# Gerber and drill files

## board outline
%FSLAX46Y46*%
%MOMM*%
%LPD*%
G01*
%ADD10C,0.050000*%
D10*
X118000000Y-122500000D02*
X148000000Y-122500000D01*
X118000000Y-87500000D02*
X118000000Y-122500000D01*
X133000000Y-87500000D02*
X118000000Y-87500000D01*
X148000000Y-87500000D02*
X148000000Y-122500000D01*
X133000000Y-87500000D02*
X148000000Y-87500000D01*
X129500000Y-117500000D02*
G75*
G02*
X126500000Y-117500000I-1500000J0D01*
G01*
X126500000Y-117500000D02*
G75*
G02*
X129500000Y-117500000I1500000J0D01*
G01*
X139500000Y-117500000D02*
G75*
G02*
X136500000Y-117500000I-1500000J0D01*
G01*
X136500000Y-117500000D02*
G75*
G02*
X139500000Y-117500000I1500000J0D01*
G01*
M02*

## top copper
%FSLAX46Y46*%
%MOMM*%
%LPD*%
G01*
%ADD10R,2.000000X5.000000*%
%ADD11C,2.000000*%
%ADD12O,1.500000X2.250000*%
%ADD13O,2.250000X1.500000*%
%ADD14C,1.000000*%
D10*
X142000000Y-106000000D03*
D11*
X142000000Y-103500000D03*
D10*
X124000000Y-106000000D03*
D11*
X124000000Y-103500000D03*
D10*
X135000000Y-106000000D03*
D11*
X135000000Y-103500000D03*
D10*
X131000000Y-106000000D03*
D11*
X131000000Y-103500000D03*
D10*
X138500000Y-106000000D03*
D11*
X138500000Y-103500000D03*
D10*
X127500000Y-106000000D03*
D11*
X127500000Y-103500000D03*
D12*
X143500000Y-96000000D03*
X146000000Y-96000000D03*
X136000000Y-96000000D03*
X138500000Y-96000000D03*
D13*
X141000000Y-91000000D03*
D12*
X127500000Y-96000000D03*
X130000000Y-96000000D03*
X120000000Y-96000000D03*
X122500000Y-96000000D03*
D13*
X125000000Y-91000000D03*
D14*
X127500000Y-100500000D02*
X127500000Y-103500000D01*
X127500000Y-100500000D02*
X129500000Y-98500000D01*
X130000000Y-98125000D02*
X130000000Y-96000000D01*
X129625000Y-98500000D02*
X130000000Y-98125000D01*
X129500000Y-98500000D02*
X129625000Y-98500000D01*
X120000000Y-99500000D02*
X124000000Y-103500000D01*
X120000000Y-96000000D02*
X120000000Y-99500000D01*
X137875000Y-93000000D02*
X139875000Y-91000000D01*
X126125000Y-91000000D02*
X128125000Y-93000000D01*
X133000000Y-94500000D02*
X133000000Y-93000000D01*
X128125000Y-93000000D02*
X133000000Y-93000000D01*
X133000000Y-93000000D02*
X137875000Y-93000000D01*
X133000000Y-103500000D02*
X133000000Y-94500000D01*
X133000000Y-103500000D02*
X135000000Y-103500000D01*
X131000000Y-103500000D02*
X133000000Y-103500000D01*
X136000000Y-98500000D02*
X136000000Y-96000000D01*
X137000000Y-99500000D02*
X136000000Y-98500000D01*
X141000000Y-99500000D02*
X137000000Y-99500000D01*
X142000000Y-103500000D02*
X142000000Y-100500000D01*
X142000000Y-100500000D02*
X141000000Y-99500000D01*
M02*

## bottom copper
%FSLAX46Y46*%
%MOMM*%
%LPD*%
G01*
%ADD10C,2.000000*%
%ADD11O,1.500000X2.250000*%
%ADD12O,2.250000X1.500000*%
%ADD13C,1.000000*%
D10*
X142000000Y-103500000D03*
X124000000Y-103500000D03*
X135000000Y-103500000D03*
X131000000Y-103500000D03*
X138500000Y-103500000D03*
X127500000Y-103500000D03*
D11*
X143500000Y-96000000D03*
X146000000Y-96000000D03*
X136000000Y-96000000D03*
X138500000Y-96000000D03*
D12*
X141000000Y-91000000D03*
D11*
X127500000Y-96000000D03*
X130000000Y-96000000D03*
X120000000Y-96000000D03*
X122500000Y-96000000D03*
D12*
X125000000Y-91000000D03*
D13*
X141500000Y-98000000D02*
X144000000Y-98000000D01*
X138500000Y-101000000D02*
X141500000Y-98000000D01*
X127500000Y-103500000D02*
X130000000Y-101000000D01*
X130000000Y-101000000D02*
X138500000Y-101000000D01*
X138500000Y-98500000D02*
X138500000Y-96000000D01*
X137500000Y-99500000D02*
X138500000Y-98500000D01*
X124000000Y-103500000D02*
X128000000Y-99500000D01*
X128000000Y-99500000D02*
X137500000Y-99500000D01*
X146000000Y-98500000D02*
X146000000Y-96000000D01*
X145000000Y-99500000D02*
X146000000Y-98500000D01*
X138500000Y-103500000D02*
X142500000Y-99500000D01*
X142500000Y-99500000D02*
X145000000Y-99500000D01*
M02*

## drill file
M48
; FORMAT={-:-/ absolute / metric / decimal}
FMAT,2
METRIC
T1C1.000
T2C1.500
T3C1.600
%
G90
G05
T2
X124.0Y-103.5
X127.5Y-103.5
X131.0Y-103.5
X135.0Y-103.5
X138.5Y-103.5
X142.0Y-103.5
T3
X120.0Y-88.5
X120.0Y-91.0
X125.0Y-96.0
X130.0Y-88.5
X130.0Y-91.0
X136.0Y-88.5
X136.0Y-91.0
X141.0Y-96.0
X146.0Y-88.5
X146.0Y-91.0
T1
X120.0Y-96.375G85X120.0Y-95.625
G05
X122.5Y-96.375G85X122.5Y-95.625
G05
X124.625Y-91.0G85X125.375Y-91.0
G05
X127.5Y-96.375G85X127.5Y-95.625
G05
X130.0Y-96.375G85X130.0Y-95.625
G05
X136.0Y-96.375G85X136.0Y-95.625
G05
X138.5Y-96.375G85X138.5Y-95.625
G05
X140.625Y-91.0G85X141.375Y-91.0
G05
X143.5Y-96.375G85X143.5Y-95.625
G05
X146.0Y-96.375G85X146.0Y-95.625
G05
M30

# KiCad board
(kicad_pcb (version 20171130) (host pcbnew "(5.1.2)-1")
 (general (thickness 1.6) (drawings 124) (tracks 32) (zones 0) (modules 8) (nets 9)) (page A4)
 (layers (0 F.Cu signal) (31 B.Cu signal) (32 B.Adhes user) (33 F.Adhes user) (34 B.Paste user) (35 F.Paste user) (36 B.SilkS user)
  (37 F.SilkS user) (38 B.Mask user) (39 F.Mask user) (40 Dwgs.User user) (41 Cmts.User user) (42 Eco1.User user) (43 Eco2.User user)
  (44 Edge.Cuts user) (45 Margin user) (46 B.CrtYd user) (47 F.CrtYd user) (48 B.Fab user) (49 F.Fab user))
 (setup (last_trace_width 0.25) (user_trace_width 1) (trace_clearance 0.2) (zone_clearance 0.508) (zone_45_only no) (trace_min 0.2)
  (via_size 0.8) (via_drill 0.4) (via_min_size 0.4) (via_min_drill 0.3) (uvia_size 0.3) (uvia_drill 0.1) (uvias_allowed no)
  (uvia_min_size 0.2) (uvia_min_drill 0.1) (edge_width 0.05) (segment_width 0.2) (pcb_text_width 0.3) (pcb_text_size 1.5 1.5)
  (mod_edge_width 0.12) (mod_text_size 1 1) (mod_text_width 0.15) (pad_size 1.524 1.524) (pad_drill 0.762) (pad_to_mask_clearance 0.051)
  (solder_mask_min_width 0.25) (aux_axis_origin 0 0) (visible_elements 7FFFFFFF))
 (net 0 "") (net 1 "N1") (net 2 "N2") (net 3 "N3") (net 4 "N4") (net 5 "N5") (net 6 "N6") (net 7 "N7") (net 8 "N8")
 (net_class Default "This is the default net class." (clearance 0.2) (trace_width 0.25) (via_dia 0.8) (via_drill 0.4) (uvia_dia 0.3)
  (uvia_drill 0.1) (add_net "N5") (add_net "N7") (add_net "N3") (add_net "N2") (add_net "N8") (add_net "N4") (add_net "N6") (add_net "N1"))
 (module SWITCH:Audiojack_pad (layer F.Cu) (at 142 103.5)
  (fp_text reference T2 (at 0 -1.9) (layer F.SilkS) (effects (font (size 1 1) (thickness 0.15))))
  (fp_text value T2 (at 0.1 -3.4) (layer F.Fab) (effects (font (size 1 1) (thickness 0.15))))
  (pad 1 smd rect (at 0 2.5 90) (size 5 2) (layers F.Cu F.Mask) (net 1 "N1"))
  (pad 1 thru_hole circle (at 0 0 90) (size 2 2) (drill 1.5) (layers *.Cu *.Mask) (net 1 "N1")))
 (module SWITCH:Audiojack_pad (layer F.Cu) (at 124 103.5)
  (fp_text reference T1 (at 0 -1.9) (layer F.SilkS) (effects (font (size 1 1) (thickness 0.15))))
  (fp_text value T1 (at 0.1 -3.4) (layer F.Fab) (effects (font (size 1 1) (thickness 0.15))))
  (pad 1 smd rect (at 0 2.5 90) (size 5 2) (layers F.Cu F.Mask) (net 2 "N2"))
  (pad 1 thru_hole circle (at 0 0 90) (size 2 2) (drill 1.5) (layers *.Cu *.Mask) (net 2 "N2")))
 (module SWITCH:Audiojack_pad (layer F.Cu) (at 135 103.5)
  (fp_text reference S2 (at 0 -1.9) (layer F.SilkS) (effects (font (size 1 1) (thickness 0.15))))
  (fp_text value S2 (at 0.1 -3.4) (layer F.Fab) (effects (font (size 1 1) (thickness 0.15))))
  (pad 1 smd rect (at 0 2.5 90) (size 5 2) (layers F.Cu F.Mask) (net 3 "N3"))
  (pad 1 thru_hole circle (at 0 0 90) (size 2 2) (drill 1.5) (layers *.Cu *.Mask) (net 3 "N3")))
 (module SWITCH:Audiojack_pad (layer F.Cu) (at 131 103.5)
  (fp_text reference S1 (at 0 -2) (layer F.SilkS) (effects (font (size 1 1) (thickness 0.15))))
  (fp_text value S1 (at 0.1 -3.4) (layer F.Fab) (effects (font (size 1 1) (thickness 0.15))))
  (pad 1 smd rect (at 0 2.5 90) (size 5 2) (layers F.Cu F.Mask) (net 3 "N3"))
  (pad 1 thru_hole circle (at 0 0 90) (size 2 2) (drill 1.5) (layers *.Cu *.Mask) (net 3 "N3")))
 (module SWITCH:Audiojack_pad (layer F.Cu) (at 138.5 103.5)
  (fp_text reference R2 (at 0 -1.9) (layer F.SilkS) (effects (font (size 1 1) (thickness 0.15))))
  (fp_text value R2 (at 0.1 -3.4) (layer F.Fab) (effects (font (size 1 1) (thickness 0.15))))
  (pad 1 smd rect (at 0 2.5 90) (size 5 2) (layers F.Cu F.Mask) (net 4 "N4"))
  (pad 1 thru_hole circle (at 0 0 90) (size 2 2) (drill 1.5) (layers *.Cu *.Mask) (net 4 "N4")))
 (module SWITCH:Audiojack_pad (layer F.Cu) (at 127.5 103.5)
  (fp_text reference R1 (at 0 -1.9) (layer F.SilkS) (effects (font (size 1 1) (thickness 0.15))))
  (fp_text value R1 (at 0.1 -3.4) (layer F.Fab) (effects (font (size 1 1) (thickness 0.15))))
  (pad 1 smd rect (at 0 2.5 90) (size 5 2) (layers F.Cu F.Mask) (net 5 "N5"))
  (pad 1 thru_hole circle (at 0 0 90) (size 2 2) (drill 1.5) (layers *.Cu *.Mask) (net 5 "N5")))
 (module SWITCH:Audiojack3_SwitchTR (layer F.Cu) (at 141 91 270)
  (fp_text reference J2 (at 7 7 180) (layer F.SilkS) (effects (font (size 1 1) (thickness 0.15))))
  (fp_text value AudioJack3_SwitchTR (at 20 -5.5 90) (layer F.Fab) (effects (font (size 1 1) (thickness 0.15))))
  (pad "" np_thru_hole circle (at 5 0 270) (size 1.6 1.6) (drill 1.6) (layers *.Cu *.Mask))
  (pad "" np_thru_hole circle (at 0 -5 270) (size 1.6 1.6) (drill 1.6) (layers *.Cu *.Mask))
  (pad "" np_thru_hole circle (at -2.5 -5 270) (size 1.6 1.6) (drill 1.6) (layers *.Cu *.Mask))
  (pad "" np_thru_hole circle (at -2.5 5 270) (size 1.6 1.6) (drill 1.6) (layers *.Cu *.Mask))
  (pad "" np_thru_hole circle (at 0 5 270) (size 1.6 1.6) (drill 1.6) (layers *.Cu *.Mask))
  (pad RN thru_hole oval (at 5 -2.5 90) (size 2.25 1.5) (drill oval 1.75 1) (layers *.Cu *.Mask) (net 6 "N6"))
  (pad R thru_hole oval (at 5 -5 90) (size 2.25 1.5) (drill oval 1.75 1) (layers *.Cu *.Mask) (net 4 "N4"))
  (pad T thru_hole oval (at 5 5 90) (size 2.25 1.5) (drill oval 1.75 1) (layers *.Cu *.Mask) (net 1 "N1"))
  (pad TN thru_hole oval (at 5 2.5 90) (size 2.25 1.5) (drill oval 1.75 1) (layers *.Cu *.Mask) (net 2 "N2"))
  (pad S thru_hole oval (at 0 0) (size 2.25 1.5) (drill oval 1.75 1) (layers *.Cu *.Mask) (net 3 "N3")))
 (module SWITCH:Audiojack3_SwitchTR (layer F.Cu) (at 125 91 270)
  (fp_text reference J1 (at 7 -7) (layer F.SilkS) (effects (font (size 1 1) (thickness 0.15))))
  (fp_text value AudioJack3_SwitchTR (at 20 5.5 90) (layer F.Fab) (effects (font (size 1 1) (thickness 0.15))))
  (pad "" np_thru_hole circle (at 5 0 270) (size 1.6 1.6) (drill 1.6) (layers *.Cu *.Mask))
  (pad "" np_thru_hole circle (at 0 -5 270) (size 1.6 1.6) (drill 1.6) (layers *.Cu *.Mask))
  (pad "" np_thru_hole circle (at -2.5 -5 270) (size 1.6 1.6) (drill 1.6) (layers *.Cu *.Mask))
  (pad "" np_thru_hole circle (at -2.5 5 270) (size 1.6 1.6) (drill 1.6) (layers *.Cu *.Mask))
  (pad "" np_thru_hole circle (at 0 5 270) (size 1.6 1.6) (drill 1.6) (layers *.Cu *.Mask))
  (pad RN thru_hole oval (at 5 -2.5 90) (size 2.25 1.5) (drill oval 1.75 1) (layers *.Cu *.Mask) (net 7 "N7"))
  (pad R thru_hole oval (at 5 -5 90) (size 2.25 1.5) (drill oval 1.75 1) (layers *.Cu *.Mask) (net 5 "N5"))
  (pad T thru_hole oval (at 5 5 90) (size 2.25 1.5) (drill oval 1.75 1) (layers *.Cu *.Mask) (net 2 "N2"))
  (pad TN thru_hole oval (at 5 2.5 90) (size 2.25 1.5) (drill oval 1.75 1) (layers *.Cu *.Mask) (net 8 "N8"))
  (pad S thru_hole oval (at 0 0) (size 2.25 1.5) (drill oval 1.75 1) (layers *.Cu *.Mask) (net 3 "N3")))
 (gr_line (start 118 122.5) (end 148 122.5) (layer Edge.Cuts) (width 0.05))
 (gr_line (start 118 87.5) (end 118 122.5) (layer Edge.Cuts) (width 0.05))
 (gr_line (start 133 87.5) (end 118 87.5) (layer Edge.Cuts) (width 0.05))
 (gr_line (start 148 87.5) (end 148 122.5) (layer Edge.Cuts) (width 0.05))
 (gr_line (start 133 87.5) (end 148 87.5) (layer Edge.Cuts) (width 0.05))
 (gr_circle (center 128 117.5) (end 129.5 117.5) (layer Edge.Cuts) (width 0.05))
 (gr_circle (center 138 117.5) (end 136.5 117.5) (layer Edge.Cuts) (width 0.05))
 (segment (start 127.5 100.5) (end 127.5 103.5) (width 1) (layer F.Cu) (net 5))
 (segment (start 127.5 100.5) (end 129.5 98.5) (width 1) (layer F.Cu) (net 5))
 (segment (start 130 98.125) (end 130 96) (width 1) (layer F.Cu) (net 5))
 (segment (start 129.625 98.5) (end 130 98.125) (width 1) (layer F.Cu) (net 5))
 (segment (start 129.5 98.5) (end 129.625 98.5) (width 1) (layer F.Cu) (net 5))
 (segment (start 141.5 98) (end 144 98) (width 1) (layer B.Cu) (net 5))
 (segment (start 138.5 101) (end 141.5 98) (width 1) (layer B.Cu) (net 5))
 (segment (start 127.5 103.5) (end 130 101) (width 1) (layer B.Cu) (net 5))
 (segment (start 130 101) (end 138.5 101) (width 1) (layer B.Cu) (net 5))
 (segment (start 120 99.5) (end 124 103.5) (width 1) (layer F.Cu) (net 2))
 (segment (start 120 96) (end 120 99.5) (width 1) (layer F.Cu) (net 2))
 (segment (start 138.5 98.5) (end 138.5 96) (width 1) (layer B.Cu) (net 2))
 (segment (start 137.5 99.5) (end 138.5 98.5) (width 1) (layer B.Cu) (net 2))
 (segment (start 124 103.5) (end 128 99.5) (width 1) (layer B.Cu) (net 2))
 (segment (start 128 99.5) (end 137.5 99.5) (width 1) (layer B.Cu) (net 2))
 (segment (start 137.875 93) (end 139.875 91) (width 1) (layer F.Cu) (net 3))
 (segment (start 126.125 91) (end 128.125 93) (width 1) (layer F.Cu) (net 3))
 (segment (start 133 94.5) (end 133 93) (width 1) (layer F.Cu) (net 3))
 (segment (start 128.125 93) (end 133 93) (width 1) (layer F.Cu) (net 3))
 (segment (start 133 93) (end 137.875 93) (width 1) (layer F.Cu) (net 3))
 (segment (start 133 103.5) (end 133 94.5) (width 1) (layer F.Cu) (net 3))
 (segment (start 133 103.5) (end 135 103.5) (width 1) (layer F.Cu) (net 3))
 (segment (start 131 103.5) (end 133 103.5) (width 1) (layer F.Cu) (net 3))
 (segment (start 146 98.5) (end 146 96) (width 1) (layer B.Cu) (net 4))
 (segment (start 145 99.5) (end 146 98.5) (width 1) (layer B.Cu) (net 4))
 (segment (start 138.5 103.5) (end 142.5 99.5) (width 1) (layer B.Cu) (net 4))
 (segment (start 142.5 99.5) (end 145 99.5) (width 1) (layer B.Cu) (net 4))
 (segment (start 136 98.5) (end 136 96) (width 1) (layer F.Cu) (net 1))
 (segment (start 137 99.5) (end 136 98.5) (width 1) (layer F.Cu) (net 1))
 (segment (start 141 99.5) (end 137 99.5) (width 1) (layer F.Cu) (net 1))
 (segment (start 142 103.5) (end 142 100.5) (width 1) (layer F.Cu) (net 1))
 (segment (start 142 100.5) (end 141 99.5) (width 1) (layer F.Cu) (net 1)))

